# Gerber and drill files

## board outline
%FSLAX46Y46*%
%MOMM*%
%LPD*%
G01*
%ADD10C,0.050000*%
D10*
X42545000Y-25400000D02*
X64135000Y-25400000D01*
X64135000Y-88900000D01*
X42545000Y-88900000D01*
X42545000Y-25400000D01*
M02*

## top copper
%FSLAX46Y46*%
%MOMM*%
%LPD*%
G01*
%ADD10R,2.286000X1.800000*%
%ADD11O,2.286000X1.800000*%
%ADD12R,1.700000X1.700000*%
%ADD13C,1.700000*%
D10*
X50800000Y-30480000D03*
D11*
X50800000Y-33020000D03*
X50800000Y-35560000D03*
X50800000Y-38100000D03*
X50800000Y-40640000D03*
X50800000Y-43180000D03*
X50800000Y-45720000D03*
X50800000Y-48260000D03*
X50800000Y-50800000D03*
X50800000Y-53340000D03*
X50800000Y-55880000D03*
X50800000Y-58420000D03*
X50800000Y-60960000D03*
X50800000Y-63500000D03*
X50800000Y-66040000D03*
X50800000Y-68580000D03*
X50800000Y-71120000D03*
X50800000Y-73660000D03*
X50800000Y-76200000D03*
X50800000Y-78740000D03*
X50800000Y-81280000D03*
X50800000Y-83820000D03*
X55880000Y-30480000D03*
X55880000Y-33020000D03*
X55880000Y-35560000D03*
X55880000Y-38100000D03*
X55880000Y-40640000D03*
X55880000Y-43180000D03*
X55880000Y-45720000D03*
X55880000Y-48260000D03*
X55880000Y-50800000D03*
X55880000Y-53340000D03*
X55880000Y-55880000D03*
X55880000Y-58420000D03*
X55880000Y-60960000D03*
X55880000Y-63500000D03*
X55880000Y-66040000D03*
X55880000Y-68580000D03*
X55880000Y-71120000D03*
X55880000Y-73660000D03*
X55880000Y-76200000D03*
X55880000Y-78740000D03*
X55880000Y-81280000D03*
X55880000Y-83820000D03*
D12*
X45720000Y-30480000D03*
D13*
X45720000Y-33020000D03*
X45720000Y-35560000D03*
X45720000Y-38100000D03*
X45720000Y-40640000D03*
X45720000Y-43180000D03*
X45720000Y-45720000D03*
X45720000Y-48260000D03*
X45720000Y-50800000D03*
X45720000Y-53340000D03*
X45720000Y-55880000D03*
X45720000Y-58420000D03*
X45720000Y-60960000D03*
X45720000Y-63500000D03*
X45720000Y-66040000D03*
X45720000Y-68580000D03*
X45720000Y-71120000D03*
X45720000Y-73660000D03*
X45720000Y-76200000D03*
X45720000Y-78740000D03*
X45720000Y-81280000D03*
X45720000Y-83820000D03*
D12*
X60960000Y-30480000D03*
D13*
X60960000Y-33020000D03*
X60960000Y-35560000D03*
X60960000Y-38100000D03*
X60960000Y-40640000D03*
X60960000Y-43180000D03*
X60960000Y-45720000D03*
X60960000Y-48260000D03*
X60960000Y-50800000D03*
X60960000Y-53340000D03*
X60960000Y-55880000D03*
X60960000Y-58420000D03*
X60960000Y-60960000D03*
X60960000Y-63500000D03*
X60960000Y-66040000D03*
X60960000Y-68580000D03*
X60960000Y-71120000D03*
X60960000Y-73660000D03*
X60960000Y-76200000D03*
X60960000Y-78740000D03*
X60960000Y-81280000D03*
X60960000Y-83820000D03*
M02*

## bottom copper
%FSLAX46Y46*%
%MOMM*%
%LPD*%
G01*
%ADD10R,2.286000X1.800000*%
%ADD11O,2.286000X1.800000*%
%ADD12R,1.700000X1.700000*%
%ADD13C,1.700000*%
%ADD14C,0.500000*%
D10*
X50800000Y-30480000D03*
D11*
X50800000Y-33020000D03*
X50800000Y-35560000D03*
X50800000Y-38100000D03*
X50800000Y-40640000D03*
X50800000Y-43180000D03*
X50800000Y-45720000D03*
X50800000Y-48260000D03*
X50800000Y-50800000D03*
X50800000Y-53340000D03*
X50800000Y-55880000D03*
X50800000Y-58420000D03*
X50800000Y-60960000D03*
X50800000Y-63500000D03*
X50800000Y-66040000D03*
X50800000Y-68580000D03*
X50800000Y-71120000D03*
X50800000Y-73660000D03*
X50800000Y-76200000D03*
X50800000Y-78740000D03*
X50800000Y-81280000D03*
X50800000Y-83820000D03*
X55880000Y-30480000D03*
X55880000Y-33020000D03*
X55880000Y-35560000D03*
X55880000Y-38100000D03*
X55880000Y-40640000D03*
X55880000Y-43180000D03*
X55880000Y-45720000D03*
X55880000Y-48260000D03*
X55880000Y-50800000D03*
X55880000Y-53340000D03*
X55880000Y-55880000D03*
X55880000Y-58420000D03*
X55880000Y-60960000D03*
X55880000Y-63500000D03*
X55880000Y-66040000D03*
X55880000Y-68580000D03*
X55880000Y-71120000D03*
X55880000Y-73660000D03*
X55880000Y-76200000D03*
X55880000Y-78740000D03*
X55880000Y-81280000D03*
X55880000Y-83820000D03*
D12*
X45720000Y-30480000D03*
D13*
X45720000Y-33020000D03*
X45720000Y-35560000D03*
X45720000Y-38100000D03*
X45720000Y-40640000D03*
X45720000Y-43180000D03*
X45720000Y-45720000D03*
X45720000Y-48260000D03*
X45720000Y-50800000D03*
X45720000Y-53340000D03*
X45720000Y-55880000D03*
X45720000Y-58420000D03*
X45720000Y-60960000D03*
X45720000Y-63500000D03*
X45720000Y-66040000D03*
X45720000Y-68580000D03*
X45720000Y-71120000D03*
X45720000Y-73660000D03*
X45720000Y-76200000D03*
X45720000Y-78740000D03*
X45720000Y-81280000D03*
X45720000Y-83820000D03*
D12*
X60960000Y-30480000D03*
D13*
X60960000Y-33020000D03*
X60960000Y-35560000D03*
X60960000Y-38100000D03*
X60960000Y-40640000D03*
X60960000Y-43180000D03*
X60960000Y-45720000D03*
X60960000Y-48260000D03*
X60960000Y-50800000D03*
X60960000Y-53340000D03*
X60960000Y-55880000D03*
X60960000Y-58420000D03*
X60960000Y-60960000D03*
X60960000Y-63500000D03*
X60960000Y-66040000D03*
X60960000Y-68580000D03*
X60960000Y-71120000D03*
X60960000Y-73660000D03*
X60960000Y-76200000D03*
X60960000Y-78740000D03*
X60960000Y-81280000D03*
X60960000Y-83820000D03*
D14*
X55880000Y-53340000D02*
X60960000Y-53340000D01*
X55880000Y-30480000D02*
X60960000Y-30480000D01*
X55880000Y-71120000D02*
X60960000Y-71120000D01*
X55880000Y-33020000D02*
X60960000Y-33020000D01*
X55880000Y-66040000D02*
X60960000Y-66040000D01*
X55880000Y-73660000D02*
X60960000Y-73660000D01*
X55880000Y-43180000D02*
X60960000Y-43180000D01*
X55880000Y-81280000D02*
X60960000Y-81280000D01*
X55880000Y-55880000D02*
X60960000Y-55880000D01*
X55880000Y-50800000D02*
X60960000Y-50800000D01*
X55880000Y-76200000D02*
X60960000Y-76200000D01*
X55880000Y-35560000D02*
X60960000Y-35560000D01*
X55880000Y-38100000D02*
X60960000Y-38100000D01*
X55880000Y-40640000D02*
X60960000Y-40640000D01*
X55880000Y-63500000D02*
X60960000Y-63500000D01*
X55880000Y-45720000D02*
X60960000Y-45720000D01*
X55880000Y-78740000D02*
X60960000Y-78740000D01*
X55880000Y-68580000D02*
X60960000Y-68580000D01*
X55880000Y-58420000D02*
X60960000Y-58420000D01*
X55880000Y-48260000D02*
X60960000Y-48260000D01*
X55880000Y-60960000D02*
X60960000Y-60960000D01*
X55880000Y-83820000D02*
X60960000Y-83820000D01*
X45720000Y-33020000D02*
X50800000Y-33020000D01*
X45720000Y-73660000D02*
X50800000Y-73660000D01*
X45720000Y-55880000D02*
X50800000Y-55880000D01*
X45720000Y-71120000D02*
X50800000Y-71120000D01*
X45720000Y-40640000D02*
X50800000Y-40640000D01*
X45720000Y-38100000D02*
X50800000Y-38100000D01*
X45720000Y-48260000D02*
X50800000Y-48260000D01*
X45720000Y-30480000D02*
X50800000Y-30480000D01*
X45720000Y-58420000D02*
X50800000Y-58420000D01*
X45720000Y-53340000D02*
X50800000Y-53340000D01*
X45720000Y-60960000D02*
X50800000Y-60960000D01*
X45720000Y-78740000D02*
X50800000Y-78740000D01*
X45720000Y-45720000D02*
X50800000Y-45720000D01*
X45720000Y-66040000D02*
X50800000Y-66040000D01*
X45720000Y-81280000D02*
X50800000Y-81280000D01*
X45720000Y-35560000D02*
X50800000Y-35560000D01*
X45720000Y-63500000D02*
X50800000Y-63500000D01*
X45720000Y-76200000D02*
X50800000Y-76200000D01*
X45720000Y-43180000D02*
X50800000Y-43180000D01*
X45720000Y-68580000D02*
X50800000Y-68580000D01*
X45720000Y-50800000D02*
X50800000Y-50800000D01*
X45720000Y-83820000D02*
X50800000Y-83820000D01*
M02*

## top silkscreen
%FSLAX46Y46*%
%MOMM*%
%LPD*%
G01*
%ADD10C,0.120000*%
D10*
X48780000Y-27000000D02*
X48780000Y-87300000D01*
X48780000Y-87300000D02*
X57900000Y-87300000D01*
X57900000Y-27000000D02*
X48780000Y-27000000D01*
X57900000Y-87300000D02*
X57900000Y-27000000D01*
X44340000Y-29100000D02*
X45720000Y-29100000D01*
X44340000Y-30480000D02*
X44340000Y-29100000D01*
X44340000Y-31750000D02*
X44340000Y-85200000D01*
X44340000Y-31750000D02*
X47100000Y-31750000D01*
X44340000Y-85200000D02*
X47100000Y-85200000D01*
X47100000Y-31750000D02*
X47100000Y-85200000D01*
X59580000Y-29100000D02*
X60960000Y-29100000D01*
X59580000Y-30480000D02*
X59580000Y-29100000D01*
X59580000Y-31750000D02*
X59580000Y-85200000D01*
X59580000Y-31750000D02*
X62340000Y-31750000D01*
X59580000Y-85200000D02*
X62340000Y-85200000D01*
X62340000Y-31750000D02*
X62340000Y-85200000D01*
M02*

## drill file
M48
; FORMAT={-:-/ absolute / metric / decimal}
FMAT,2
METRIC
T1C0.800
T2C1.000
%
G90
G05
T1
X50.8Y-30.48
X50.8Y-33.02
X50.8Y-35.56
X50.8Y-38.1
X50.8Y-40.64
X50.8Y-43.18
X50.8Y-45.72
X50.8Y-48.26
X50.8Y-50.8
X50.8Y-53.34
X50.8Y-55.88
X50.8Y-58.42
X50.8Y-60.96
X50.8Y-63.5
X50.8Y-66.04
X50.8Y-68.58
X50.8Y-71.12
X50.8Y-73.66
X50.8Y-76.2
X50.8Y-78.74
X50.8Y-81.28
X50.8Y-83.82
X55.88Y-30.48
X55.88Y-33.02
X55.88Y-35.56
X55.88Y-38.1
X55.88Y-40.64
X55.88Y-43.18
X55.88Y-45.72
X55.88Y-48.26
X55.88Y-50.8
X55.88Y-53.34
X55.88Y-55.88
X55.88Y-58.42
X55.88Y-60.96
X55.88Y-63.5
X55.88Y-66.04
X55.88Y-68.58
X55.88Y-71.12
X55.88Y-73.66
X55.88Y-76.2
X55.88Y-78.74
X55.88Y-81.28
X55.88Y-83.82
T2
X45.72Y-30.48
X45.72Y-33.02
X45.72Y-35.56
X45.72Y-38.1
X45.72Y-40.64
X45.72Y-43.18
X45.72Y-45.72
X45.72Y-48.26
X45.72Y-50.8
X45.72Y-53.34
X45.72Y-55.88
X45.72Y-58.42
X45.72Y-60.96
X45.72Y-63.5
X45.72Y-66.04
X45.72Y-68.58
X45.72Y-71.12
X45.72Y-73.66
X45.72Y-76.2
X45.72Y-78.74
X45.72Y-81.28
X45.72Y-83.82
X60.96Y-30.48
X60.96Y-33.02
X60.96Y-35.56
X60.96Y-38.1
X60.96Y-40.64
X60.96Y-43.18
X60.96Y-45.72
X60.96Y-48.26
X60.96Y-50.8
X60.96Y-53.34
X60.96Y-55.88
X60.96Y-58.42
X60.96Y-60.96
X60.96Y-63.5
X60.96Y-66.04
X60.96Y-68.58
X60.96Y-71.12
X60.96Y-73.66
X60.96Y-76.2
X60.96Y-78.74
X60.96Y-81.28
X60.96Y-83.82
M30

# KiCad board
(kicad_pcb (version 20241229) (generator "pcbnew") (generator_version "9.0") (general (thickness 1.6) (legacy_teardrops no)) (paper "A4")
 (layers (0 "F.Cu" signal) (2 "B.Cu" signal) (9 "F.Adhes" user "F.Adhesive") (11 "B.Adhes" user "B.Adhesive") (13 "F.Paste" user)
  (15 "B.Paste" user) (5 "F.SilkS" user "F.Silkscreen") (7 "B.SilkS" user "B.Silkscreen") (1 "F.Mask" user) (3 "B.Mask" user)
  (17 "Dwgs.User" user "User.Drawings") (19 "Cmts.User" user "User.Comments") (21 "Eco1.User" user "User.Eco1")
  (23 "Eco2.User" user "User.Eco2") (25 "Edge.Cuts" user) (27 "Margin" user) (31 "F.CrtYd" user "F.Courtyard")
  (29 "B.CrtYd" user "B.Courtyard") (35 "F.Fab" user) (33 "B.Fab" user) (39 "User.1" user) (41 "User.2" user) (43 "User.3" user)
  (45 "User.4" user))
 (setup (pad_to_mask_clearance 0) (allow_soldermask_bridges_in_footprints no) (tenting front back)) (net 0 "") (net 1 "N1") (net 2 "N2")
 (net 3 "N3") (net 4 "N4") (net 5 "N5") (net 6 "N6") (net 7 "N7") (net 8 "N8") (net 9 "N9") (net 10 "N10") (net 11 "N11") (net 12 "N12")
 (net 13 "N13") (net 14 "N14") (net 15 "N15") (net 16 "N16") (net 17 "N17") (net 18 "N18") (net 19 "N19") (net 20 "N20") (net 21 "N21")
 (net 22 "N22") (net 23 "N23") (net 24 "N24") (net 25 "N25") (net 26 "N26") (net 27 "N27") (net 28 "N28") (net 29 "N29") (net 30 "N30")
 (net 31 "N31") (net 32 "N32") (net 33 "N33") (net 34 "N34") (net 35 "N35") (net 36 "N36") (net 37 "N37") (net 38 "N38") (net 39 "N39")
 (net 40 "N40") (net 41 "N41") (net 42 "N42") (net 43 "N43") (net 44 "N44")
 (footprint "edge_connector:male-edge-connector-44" (layer "F.Cu") (at 50.8 30.48)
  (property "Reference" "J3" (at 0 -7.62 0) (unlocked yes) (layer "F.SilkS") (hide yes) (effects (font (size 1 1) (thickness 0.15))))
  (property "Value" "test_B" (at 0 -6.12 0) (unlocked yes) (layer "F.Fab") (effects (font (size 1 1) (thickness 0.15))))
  (fp_line (start -2.02 -3.48) (end -2.02 56.82) (stroke (width 0.12) (type solid)) (layer "F.SilkS"))
  (fp_line (start -2.02 56.82) (end 7.1 56.82) (stroke (width 0.12) (type solid)) (layer "F.SilkS"))
  (fp_line (start 7.1 -3.48) (end -2.02 -3.48) (stroke (width 0.12) (type solid)) (layer "F.SilkS"))
  (fp_line (start 7.1 56.82) (end 7.1 -3.48) (stroke (width 0.12) (type solid)) (layer "F.SilkS"))
  (pad "1" thru_hole rect (at 0 0) (size 2.286 1.8) (drill 0.8) (layers "*.Cu" "*.Mask") (remove_unused_layers yes) (keep_end_layers yes)
   (zone_layer_connections) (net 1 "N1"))
  (pad "2" thru_hole oval (at 0 2.54) (size 2.286 1.8) (drill 0.8) (layers "*.Cu" "*.Mask") (remove_unused_layers no) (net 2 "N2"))
  (pad "3" thru_hole oval (at 0 5.08) (size 2.286 1.8) (drill 0.8) (layers "*.Cu" "*.Mask") (remove_unused_layers no) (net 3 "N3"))
  (pad "4" thru_hole oval (at 0 7.62) (size 2.286 1.8) (drill 0.8) (layers "*.Cu" "*.Mask") (remove_unused_layers no) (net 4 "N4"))
  (pad "5" thru_hole oval (at 0 10.16) (size 2.286 1.8) (drill 0.8) (layers "*.Cu" "*.Mask") (remove_unused_layers no) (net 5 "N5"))
  (pad "6" thru_hole oval (at 0 12.7) (size 2.286 1.8) (drill 0.8) (layers "*.Cu" "*.Mask") (remove_unused_layers no) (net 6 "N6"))
  (pad "7" thru_hole oval (at 0 15.24) (size 2.286 1.8) (drill 0.8) (layers "*.Cu" "*.Mask") (remove_unused_layers no) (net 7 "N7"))
  (pad "8" thru_hole oval (at 0 17.78) (size 2.286 1.8) (drill 0.8) (layers "*.Cu" "*.Mask") (remove_unused_layers no) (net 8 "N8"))
  (pad "9" thru_hole oval (at 0 20.32) (size 2.286 1.8) (drill 0.8) (layers "*.Cu" "*.Mask") (remove_unused_layers no) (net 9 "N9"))
  (pad "10" thru_hole oval (at 0 22.86) (size 2.286 1.8) (drill 0.8) (layers "*.Cu" "*.Mask") (remove_unused_layers no) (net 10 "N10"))
  (pad "11" thru_hole oval (at 0 25.4) (size 2.286 1.8) (drill 0.8) (layers "*.Cu" "*.Mask") (remove_unused_layers no) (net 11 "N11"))
  (pad "12" thru_hole oval (at 0 27.94) (size 2.286 1.8) (drill 0.8) (layers "*.Cu" "*.Mask") (remove_unused_layers no) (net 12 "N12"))
  (pad "13" thru_hole oval (at 0 30.48) (size 2.286 1.8) (drill 0.8) (layers "*.Cu" "*.Mask") (remove_unused_layers no) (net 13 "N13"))
  (pad "14" thru_hole oval (at 0 33.02) (size 2.286 1.8) (drill 0.8) (layers "*.Cu" "*.Mask") (remove_unused_layers no) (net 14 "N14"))
  (pad "15" thru_hole oval (at 0 35.56) (size 2.286 1.8) (drill 0.8) (layers "*.Cu" "*.Mask") (remove_unused_layers no) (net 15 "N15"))
  (pad "16" thru_hole oval (at 0 38.1) (size 2.286 1.8) (drill 0.8) (layers "*.Cu" "*.Mask") (remove_unused_layers no) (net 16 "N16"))
  (pad "17" thru_hole oval (at 0 40.64) (size 2.286 1.8) (drill 0.8) (layers "*.Cu" "*.Mask") (remove_unused_layers no) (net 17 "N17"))
  (pad "18" thru_hole oval (at 0 43.18) (size 2.286 1.8) (drill 0.8) (layers "*.Cu" "*.Mask") (remove_unused_layers no) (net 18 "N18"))
  (pad "19" thru_hole oval (at 0 45.72) (size 2.286 1.8) (drill 0.8) (layers "*.Cu" "*.Mask") (remove_unused_layers no) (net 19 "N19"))
  (pad "20" thru_hole oval (at 0 48.26) (size 2.286 1.8) (drill 0.8) (layers "*.Cu" "*.Mask") (remove_unused_layers no) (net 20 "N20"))
  (pad "21" thru_hole oval (at 0 50.8) (size 2.286 1.8) (drill 0.8) (layers "*.Cu" "*.Mask") (remove_unused_layers no) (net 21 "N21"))
  (pad "22" thru_hole oval (at 0 53.34) (size 2.286 1.8) (drill 0.8) (layers "*.Cu" "*.Mask") (remove_unused_layers no) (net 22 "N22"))
  (pad "23" thru_hole oval (at 5.08 0) (size 2.286 1.8) (drill 0.8) (layers "*.Cu" "*.Mask") (remove_unused_layers no) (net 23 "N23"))
  (pad "24" thru_hole oval (at 5.08 2.54) (size 2.286 1.8) (drill 0.8) (layers "*.Cu" "*.Mask") (remove_unused_layers no) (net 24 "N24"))
  (pad "25" thru_hole oval (at 5.08 5.08) (size 2.286 1.8) (drill 0.8) (layers "*.Cu" "*.Mask") (remove_unused_layers no) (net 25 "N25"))
  (pad "26" thru_hole oval (at 5.08 7.62) (size 2.286 1.8) (drill 0.8) (layers "*.Cu" "*.Mask") (remove_unused_layers no) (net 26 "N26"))
  (pad "27" thru_hole oval (at 5.08 10.16) (size 2.286 1.8) (drill 0.8) (layers "*.Cu" "*.Mask") (remove_unused_layers no) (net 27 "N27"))
  (pad "28" thru_hole oval (at 5.08 12.7) (size 2.286 1.8) (drill 0.8) (layers "*.Cu" "*.Mask") (remove_unused_layers no) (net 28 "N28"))
  (pad "29" thru_hole oval (at 5.08 15.24) (size 2.286 1.8) (drill 0.8) (layers "*.Cu" "*.Mask") (remove_unused_layers no) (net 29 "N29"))
  (pad "30" thru_hole oval (at 5.08 17.78) (size 2.286 1.8) (drill 0.8) (layers "*.Cu" "*.Mask") (remove_unused_layers no) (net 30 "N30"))
  (pad "31" thru_hole oval (at 5.08 20.32) (size 2.286 1.8) (drill 0.8) (layers "*.Cu" "*.Mask") (remove_unused_layers no) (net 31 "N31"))
  (pad "32" thru_hole oval (at 5.08 22.86) (size 2.286 1.8) (drill 0.8) (layers "*.Cu" "*.Mask") (remove_unused_layers no) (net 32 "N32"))
  (pad "33" thru_hole oval (at 5.08 25.4) (size 2.286 1.8) (drill 0.8) (layers "*.Cu" "*.Mask") (remove_unused_layers no) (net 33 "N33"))
  (pad "34" thru_hole oval (at 5.08 27.94) (size 2.286 1.8) (drill 0.8) (layers "*.Cu" "*.Mask") (remove_unused_layers no) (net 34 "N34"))
  (pad "35" thru_hole oval (at 5.08 30.48) (size 2.286 1.8) (drill 0.8) (layers "*.Cu" "*.Mask") (remove_unused_layers no) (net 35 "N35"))
  (pad "36" thru_hole oval (at 5.08 33.02) (size 2.286 1.8) (drill 0.8) (layers "*.Cu" "*.Mask") (remove_unused_layers no) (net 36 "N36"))
  (pad "37" thru_hole oval (at 5.08 35.56) (size 2.286 1.8) (drill 0.8) (layers "*.Cu" "*.Mask") (remove_unused_layers no) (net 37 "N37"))
  (pad "38" thru_hole oval (at 5.08 38.1) (size 2.286 1.8) (drill 0.8) (layers "*.Cu" "*.Mask") (remove_unused_layers no) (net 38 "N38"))
  (pad "39" thru_hole oval (at 5.08 40.64) (size 2.286 1.8) (drill 0.8) (layers "*.Cu" "*.Mask") (remove_unused_layers no) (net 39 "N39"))
  (pad "40" thru_hole oval (at 5.08 43.18) (size 2.286 1.8) (drill 0.8) (layers "*.Cu" "*.Mask") (remove_unused_layers no) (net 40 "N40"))
  (pad "41" thru_hole oval (at 5.08 45.72) (size 2.286 1.8) (drill 0.8) (layers "*.Cu" "*.Mask") (remove_unused_layers no) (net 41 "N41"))
  (pad "42" thru_hole oval (at 5.08 48.26) (size 2.286 1.8) (drill 0.8) (layers "*.Cu" "*.Mask") (remove_unused_layers no) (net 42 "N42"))
  (pad "43" thru_hole oval (at 5.08 50.8) (size 2.286 1.8) (drill 0.8) (layers "*.Cu" "*.Mask") (remove_unused_layers no) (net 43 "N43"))
  (pad "44" thru_hole oval (at 5.08 53.34) (size 2.286 1.8) (drill 0.8) (layers "*.Cu" "*.Mask") (remove_unused_layers no) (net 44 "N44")))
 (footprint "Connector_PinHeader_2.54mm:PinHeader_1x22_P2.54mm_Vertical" (layer "F.Cu") (at 45.72 30.48)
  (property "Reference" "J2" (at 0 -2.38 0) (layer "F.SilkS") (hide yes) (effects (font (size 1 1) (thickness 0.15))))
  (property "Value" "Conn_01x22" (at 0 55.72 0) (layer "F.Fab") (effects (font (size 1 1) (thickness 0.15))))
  (fp_line (start -1.38 -1.38) (end 0 -1.38) (stroke (width 0.12) (type solid)) (layer "F.SilkS"))
  (fp_line (start -1.38 0) (end -1.38 -1.38) (stroke (width 0.12) (type solid)) (layer "F.SilkS"))
  (fp_line (start -1.38 1.27) (end -1.38 54.72) (stroke (width 0.12) (type solid)) (layer "F.SilkS"))
  (fp_line (start -1.38 1.27) (end 1.38 1.27) (stroke (width 0.12) (type solid)) (layer "F.SilkS"))
  (fp_line (start -1.38 54.72) (end 1.38 54.72) (stroke (width 0.12) (type solid)) (layer "F.SilkS"))
  (fp_line (start 1.38 1.27) (end 1.38 54.72) (stroke (width 0.12) (type solid)) (layer "F.SilkS"))
  (pad "1" thru_hole rect (at 0 0) (size 1.7 1.7) (drill 1) (layers "*.Cu" "*.Mask") (remove_unused_layers no) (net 1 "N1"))
  (pad "2" thru_hole circle (at 0 2.54) (size 1.7 1.7) (drill 1) (layers "*.Cu" "*.Mask") (remove_unused_layers no) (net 2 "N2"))
  (pad "3" thru_hole circle (at 0 5.08) (size 1.7 1.7) (drill 1) (layers "*.Cu" "*.Mask") (remove_unused_layers no) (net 3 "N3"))
  (pad "4" thru_hole circle (at 0 7.62) (size 1.7 1.7) (drill 1) (layers "*.Cu" "*.Mask") (remove_unused_layers no) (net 4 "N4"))
  (pad "5" thru_hole circle (at 0 10.16) (size 1.7 1.7) (drill 1) (layers "*.Cu" "*.Mask") (remove_unused_layers no) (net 5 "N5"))
  (pad "6" thru_hole circle (at 0 12.7) (size 1.7 1.7) (drill 1) (layers "*.Cu" "*.Mask") (remove_unused_layers no) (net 6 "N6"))
  (pad "7" thru_hole circle (at 0 15.24) (size 1.7 1.7) (drill 1) (layers "*.Cu" "*.Mask") (remove_unused_layers no) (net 7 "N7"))
  (pad "8" thru_hole circle (at 0 17.78) (size 1.7 1.7) (drill 1) (layers "*.Cu" "*.Mask") (remove_unused_layers no) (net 8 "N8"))
  (pad "9" thru_hole circle (at 0 20.32) (size 1.7 1.7) (drill 1) (layers "*.Cu" "*.Mask") (remove_unused_layers no) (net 9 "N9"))
  (pad "10" thru_hole circle (at 0 22.86) (size 1.7 1.7) (drill 1) (layers "*.Cu" "*.Mask") (remove_unused_layers no) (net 10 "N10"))
  (pad "11" thru_hole circle (at 0 25.4) (size 1.7 1.7) (drill 1) (layers "*.Cu" "*.Mask") (remove_unused_layers no) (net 11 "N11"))
  (pad "12" thru_hole circle (at 0 27.94) (size 1.7 1.7) (drill 1) (layers "*.Cu" "*.Mask") (remove_unused_layers no) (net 12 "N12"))
  (pad "13" thru_hole circle (at 0 30.48) (size 1.7 1.7) (drill 1) (layers "*.Cu" "*.Mask") (remove_unused_layers no) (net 13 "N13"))
  (pad "14" thru_hole circle (at 0 33.02) (size 1.7 1.7) (drill 1) (layers "*.Cu" "*.Mask") (remove_unused_layers no) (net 14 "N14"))
  (pad "15" thru_hole circle (at 0 35.56) (size 1.7 1.7) (drill 1) (layers "*.Cu" "*.Mask") (remove_unused_layers no) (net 15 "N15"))
  (pad "16" thru_hole circle (at 0 38.1) (size 1.7 1.7) (drill 1) (layers "*.Cu" "*.Mask") (remove_unused_layers no) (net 16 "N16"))
  (pad "17" thru_hole circle (at 0 40.64) (size 1.7 1.7) (drill 1) (layers "*.Cu" "*.Mask") (remove_unused_layers no) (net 17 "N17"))
  (pad "18" thru_hole circle (at 0 43.18) (size 1.7 1.7) (drill 1) (layers "*.Cu" "*.Mask") (remove_unused_layers no) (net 18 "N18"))
  (pad "19" thru_hole circle (at 0 45.72) (size 1.7 1.7) (drill 1) (layers "*.Cu" "*.Mask") (remove_unused_layers no) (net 19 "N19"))
  (pad "20" thru_hole circle (at 0 48.26) (size 1.7 1.7) (drill 1) (layers "*.Cu" "*.Mask") (remove_unused_layers no) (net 20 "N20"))
  (pad "21" thru_hole circle (at 0 50.8) (size 1.7 1.7) (drill 1) (layers "*.Cu" "*.Mask") (remove_unused_layers no) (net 21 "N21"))
  (pad "22" thru_hole circle (at 0 53.34) (size 1.7 1.7) (drill 1) (layers "*.Cu" "*.Mask") (remove_unused_layers no) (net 22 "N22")))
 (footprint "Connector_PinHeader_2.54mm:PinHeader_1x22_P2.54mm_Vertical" (layer "F.Cu") (at 60.96 30.48)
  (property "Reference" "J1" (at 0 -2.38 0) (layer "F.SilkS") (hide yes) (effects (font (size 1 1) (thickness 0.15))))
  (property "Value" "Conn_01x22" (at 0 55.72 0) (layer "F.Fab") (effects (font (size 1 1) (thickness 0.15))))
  (fp_line (start -1.38 -1.38) (end 0 -1.38) (stroke (width 0.12) (type solid)) (layer "F.SilkS"))
  (fp_line (start -1.38 0) (end -1.38 -1.38) (stroke (width 0.12) (type solid)) (layer "F.SilkS"))
  (fp_line (start -1.38 1.27) (end -1.38 54.72) (stroke (width 0.12) (type solid)) (layer "F.SilkS"))
  (fp_line (start -1.38 1.27) (end 1.38 1.27) (stroke (width 0.12) (type solid)) (layer "F.SilkS"))
  (fp_line (start -1.38 54.72) (end 1.38 54.72) (stroke (width 0.12) (type solid)) (layer "F.SilkS"))
  (fp_line (start 1.38 1.27) (end 1.38 54.72) (stroke (width 0.12) (type solid)) (layer "F.SilkS"))
  (pad "1" thru_hole rect (at 0 0) (size 1.7 1.7) (drill 1) (layers "*.Cu" "*.Mask") (remove_unused_layers no) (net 23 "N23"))
  (pad "2" thru_hole circle (at 0 2.54) (size 1.7 1.7) (drill 1) (layers "*.Cu" "*.Mask") (remove_unused_layers no) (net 24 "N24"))
  (pad "3" thru_hole circle (at 0 5.08) (size 1.7 1.7) (drill 1) (layers "*.Cu" "*.Mask") (remove_unused_layers no) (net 25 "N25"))
  (pad "4" thru_hole circle (at 0 7.62) (size 1.7 1.7) (drill 1) (layers "*.Cu" "*.Mask") (remove_unused_layers no) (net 26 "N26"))
  (pad "5" thru_hole circle (at 0 10.16) (size 1.7 1.7) (drill 1) (layers "*.Cu" "*.Mask") (remove_unused_layers no) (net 27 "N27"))
  (pad "6" thru_hole circle (at 0 12.7) (size 1.7 1.7) (drill 1) (layers "*.Cu" "*.Mask") (remove_unused_layers no) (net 28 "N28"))
  (pad "7" thru_hole circle (at 0 15.24) (size 1.7 1.7) (drill 1) (layers "*.Cu" "*.Mask") (remove_unused_layers no) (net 29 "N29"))
  (pad "8" thru_hole circle (at 0 17.78) (size 1.7 1.7) (drill 1) (layers "*.Cu" "*.Mask") (remove_unused_layers no) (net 30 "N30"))
  (pad "9" thru_hole circle (at 0 20.32) (size 1.7 1.7) (drill 1) (layers "*.Cu" "*.Mask") (remove_unused_layers no) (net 31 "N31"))
  (pad "10" thru_hole circle (at 0 22.86) (size 1.7 1.7) (drill 1) (layers "*.Cu" "*.Mask") (remove_unused_layers no) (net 32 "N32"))
  (pad "11" thru_hole circle (at 0 25.4) (size 1.7 1.7) (drill 1) (layers "*.Cu" "*.Mask") (remove_unused_layers no) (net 33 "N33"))
  (pad "12" thru_hole circle (at 0 27.94) (size 1.7 1.7) (drill 1) (layers "*.Cu" "*.Mask") (remove_unused_layers no) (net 34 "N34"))
  (pad "13" thru_hole circle (at 0 30.48) (size 1.7 1.7) (drill 1) (layers "*.Cu" "*.Mask") (remove_unused_layers no) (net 35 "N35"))
  (pad "14" thru_hole circle (at 0 33.02) (size 1.7 1.7) (drill 1) (layers "*.Cu" "*.Mask") (remove_unused_layers no) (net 36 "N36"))
  (pad "15" thru_hole circle (at 0 35.56) (size 1.7 1.7) (drill 1) (layers "*.Cu" "*.Mask") (remove_unused_layers no) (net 37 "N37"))
  (pad "16" thru_hole circle (at 0 38.1) (size 1.7 1.7) (drill 1) (layers "*.Cu" "*.Mask") (remove_unused_layers no) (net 38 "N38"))
  (pad "17" thru_hole circle (at 0 40.64) (size 1.7 1.7) (drill 1) (layers "*.Cu" "*.Mask") (remove_unused_layers no) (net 39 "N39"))
  (pad "18" thru_hole circle (at 0 43.18) (size 1.7 1.7) (drill 1) (layers "*.Cu" "*.Mask") (remove_unused_layers no) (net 40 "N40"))
  (pad "19" thru_hole circle (at 0 45.72) (size 1.7 1.7) (drill 1) (layers "*.Cu" "*.Mask") (remove_unused_layers no) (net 41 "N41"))
  (pad "20" thru_hole circle (at 0 48.26) (size 1.7 1.7) (drill 1) (layers "*.Cu" "*.Mask") (remove_unused_layers no) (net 42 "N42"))
  (pad "21" thru_hole circle (at 0 50.8) (size 1.7 1.7) (drill 1) (layers "*.Cu" "*.Mask") (remove_unused_layers no) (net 43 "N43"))
  (pad "22" thru_hole circle (at 0 53.34) (size 1.7 1.7) (drill 1) (layers "*.Cu" "*.Mask") (remove_unused_layers no) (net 44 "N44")))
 (gr_rect (start 42.545 25.4) (end 64.135 88.9) (stroke (width 0.05) (type default)) (fill no) (layer "Edge.Cuts"))
 (segment (start 55.88 53.34) (end 60.96 53.34) (width 0.5) (layer "B.Cu") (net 32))
 (segment (start 55.88 30.48) (end 60.96 30.48) (width 0.5) (layer "B.Cu") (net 23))
 (segment (start 55.88 71.12) (end 60.96 71.12) (width 0.5) (layer "B.Cu") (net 39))
 (segment (start 55.88 33.02) (end 60.96 33.02) (width 0.5) (layer "B.Cu") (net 24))
 (segment (start 55.88 66.04) (end 60.96 66.04) (width 0.5) (layer "B.Cu") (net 37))
 (segment (start 55.88 73.66) (end 60.96 73.66) (width 0.5) (layer "B.Cu") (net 40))
 (segment (start 55.88 43.18) (end 60.96 43.18) (width 0.5) (layer "B.Cu") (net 28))
 (segment (start 55.88 81.28) (end 60.96 81.28) (width 0.5) (layer "B.Cu") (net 43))
 (segment (start 55.88 55.88) (end 60.96 55.88) (width 0.5) (layer "B.Cu") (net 33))
 (segment (start 55.88 50.8) (end 60.96 50.8) (width 0.5) (layer "B.Cu") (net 31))
 (segment (start 55.88 76.2) (end 60.96 76.2) (width 0.5) (layer "B.Cu") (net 41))
 (segment (start 55.88 35.56) (end 60.96 35.56) (width 0.5) (layer "B.Cu") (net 25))
 (segment (start 55.88 38.1) (end 60.96 38.1) (width 0.5) (layer "B.Cu") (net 26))
 (segment (start 55.88 40.64) (end 60.96 40.64) (width 0.5) (layer "B.Cu") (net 27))
 (segment (start 55.88 63.5) (end 60.96 63.5) (width 0.5) (layer "B.Cu") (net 36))
 (segment (start 55.88 45.72) (end 60.96 45.72) (width 0.5) (layer "B.Cu") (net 29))
 (segment (start 55.88 78.74) (end 60.96 78.74) (width 0.5) (layer "B.Cu") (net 42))
 (segment (start 55.88 68.58) (end 60.96 68.58) (width 0.5) (layer "B.Cu") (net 38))
 (segment (start 55.88 58.42) (end 60.96 58.42) (width 0.5) (layer "B.Cu") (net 34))
 (segment (start 55.88 48.26) (end 60.96 48.26) (width 0.5) (layer "B.Cu") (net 30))
 (segment (start 55.88 60.96) (end 60.96 60.96) (width 0.5) (layer "B.Cu") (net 35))
 (segment (start 55.88 83.82) (end 60.96 83.82) (width 0.5) (layer "B.Cu") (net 44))
 (segment (start 45.72 33.02) (end 50.8 33.02) (width 0.5) (layer "B.Cu") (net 2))
 (segment (start 45.72 73.66) (end 50.8 73.66) (width 0.5) (layer "B.Cu") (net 18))
 (segment (start 45.72 55.88) (end 50.8 55.88) (width 0.5) (layer "B.Cu") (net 11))
 (segment (start 45.72 71.12) (end 50.8 71.12) (width 0.5) (layer "B.Cu") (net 17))
 (segment (start 45.72 40.64) (end 50.8 40.64) (width 0.5) (layer "B.Cu") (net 5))
 (segment (start 45.72 38.1) (end 50.8 38.1) (width 0.5) (layer "B.Cu") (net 4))
 (segment (start 45.72 48.26) (end 50.8 48.26) (width 0.5) (layer "B.Cu") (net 8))
 (segment (start 45.72 30.48) (end 50.8 30.48) (width 0.5) (layer "B.Cu") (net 1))
 (segment (start 45.72 58.42) (end 50.8 58.42) (width 0.5) (layer "B.Cu") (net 12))
 (segment (start 45.72 53.34) (end 50.8 53.34) (width 0.5) (layer "B.Cu") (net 10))
 (segment (start 45.72 60.96) (end 50.8 60.96) (width 0.5) (layer "B.Cu") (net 13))
 (segment (start 45.72 78.74) (end 50.8 78.74) (width 0.5) (layer "B.Cu") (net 20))
 (segment (start 45.72 45.72) (end 50.8 45.72) (width 0.5) (layer "B.Cu") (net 7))
 (segment (start 45.72 66.04) (end 50.8 66.04) (width 0.5) (layer "B.Cu") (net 15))
 (segment (start 45.72 81.28) (end 50.8 81.28) (width 0.5) (layer "B.Cu") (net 21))
 (segment (start 45.72 35.56) (end 50.8 35.56) (width 0.5) (layer "B.Cu") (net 3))
 (segment (start 45.72 63.5) (end 50.8 63.5) (width 0.5) (layer "B.Cu") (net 14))
 (segment (start 45.72 76.2) (end 50.8 76.2) (width 0.5) (layer "B.Cu") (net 19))
 (segment (start 45.72 43.18) (end 50.8 43.18) (width 0.5) (layer "B.Cu") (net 6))
 (segment (start 45.72 68.58) (end 50.8 68.58) (width 0.5) (layer "B.Cu") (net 16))
 (segment (start 45.72 50.8) (end 50.8 50.8) (width 0.5) (layer "B.Cu") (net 9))
 (segment (start 45.72 83.82) (end 50.8 83.82) (width 0.5) (layer "B.Cu") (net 22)))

